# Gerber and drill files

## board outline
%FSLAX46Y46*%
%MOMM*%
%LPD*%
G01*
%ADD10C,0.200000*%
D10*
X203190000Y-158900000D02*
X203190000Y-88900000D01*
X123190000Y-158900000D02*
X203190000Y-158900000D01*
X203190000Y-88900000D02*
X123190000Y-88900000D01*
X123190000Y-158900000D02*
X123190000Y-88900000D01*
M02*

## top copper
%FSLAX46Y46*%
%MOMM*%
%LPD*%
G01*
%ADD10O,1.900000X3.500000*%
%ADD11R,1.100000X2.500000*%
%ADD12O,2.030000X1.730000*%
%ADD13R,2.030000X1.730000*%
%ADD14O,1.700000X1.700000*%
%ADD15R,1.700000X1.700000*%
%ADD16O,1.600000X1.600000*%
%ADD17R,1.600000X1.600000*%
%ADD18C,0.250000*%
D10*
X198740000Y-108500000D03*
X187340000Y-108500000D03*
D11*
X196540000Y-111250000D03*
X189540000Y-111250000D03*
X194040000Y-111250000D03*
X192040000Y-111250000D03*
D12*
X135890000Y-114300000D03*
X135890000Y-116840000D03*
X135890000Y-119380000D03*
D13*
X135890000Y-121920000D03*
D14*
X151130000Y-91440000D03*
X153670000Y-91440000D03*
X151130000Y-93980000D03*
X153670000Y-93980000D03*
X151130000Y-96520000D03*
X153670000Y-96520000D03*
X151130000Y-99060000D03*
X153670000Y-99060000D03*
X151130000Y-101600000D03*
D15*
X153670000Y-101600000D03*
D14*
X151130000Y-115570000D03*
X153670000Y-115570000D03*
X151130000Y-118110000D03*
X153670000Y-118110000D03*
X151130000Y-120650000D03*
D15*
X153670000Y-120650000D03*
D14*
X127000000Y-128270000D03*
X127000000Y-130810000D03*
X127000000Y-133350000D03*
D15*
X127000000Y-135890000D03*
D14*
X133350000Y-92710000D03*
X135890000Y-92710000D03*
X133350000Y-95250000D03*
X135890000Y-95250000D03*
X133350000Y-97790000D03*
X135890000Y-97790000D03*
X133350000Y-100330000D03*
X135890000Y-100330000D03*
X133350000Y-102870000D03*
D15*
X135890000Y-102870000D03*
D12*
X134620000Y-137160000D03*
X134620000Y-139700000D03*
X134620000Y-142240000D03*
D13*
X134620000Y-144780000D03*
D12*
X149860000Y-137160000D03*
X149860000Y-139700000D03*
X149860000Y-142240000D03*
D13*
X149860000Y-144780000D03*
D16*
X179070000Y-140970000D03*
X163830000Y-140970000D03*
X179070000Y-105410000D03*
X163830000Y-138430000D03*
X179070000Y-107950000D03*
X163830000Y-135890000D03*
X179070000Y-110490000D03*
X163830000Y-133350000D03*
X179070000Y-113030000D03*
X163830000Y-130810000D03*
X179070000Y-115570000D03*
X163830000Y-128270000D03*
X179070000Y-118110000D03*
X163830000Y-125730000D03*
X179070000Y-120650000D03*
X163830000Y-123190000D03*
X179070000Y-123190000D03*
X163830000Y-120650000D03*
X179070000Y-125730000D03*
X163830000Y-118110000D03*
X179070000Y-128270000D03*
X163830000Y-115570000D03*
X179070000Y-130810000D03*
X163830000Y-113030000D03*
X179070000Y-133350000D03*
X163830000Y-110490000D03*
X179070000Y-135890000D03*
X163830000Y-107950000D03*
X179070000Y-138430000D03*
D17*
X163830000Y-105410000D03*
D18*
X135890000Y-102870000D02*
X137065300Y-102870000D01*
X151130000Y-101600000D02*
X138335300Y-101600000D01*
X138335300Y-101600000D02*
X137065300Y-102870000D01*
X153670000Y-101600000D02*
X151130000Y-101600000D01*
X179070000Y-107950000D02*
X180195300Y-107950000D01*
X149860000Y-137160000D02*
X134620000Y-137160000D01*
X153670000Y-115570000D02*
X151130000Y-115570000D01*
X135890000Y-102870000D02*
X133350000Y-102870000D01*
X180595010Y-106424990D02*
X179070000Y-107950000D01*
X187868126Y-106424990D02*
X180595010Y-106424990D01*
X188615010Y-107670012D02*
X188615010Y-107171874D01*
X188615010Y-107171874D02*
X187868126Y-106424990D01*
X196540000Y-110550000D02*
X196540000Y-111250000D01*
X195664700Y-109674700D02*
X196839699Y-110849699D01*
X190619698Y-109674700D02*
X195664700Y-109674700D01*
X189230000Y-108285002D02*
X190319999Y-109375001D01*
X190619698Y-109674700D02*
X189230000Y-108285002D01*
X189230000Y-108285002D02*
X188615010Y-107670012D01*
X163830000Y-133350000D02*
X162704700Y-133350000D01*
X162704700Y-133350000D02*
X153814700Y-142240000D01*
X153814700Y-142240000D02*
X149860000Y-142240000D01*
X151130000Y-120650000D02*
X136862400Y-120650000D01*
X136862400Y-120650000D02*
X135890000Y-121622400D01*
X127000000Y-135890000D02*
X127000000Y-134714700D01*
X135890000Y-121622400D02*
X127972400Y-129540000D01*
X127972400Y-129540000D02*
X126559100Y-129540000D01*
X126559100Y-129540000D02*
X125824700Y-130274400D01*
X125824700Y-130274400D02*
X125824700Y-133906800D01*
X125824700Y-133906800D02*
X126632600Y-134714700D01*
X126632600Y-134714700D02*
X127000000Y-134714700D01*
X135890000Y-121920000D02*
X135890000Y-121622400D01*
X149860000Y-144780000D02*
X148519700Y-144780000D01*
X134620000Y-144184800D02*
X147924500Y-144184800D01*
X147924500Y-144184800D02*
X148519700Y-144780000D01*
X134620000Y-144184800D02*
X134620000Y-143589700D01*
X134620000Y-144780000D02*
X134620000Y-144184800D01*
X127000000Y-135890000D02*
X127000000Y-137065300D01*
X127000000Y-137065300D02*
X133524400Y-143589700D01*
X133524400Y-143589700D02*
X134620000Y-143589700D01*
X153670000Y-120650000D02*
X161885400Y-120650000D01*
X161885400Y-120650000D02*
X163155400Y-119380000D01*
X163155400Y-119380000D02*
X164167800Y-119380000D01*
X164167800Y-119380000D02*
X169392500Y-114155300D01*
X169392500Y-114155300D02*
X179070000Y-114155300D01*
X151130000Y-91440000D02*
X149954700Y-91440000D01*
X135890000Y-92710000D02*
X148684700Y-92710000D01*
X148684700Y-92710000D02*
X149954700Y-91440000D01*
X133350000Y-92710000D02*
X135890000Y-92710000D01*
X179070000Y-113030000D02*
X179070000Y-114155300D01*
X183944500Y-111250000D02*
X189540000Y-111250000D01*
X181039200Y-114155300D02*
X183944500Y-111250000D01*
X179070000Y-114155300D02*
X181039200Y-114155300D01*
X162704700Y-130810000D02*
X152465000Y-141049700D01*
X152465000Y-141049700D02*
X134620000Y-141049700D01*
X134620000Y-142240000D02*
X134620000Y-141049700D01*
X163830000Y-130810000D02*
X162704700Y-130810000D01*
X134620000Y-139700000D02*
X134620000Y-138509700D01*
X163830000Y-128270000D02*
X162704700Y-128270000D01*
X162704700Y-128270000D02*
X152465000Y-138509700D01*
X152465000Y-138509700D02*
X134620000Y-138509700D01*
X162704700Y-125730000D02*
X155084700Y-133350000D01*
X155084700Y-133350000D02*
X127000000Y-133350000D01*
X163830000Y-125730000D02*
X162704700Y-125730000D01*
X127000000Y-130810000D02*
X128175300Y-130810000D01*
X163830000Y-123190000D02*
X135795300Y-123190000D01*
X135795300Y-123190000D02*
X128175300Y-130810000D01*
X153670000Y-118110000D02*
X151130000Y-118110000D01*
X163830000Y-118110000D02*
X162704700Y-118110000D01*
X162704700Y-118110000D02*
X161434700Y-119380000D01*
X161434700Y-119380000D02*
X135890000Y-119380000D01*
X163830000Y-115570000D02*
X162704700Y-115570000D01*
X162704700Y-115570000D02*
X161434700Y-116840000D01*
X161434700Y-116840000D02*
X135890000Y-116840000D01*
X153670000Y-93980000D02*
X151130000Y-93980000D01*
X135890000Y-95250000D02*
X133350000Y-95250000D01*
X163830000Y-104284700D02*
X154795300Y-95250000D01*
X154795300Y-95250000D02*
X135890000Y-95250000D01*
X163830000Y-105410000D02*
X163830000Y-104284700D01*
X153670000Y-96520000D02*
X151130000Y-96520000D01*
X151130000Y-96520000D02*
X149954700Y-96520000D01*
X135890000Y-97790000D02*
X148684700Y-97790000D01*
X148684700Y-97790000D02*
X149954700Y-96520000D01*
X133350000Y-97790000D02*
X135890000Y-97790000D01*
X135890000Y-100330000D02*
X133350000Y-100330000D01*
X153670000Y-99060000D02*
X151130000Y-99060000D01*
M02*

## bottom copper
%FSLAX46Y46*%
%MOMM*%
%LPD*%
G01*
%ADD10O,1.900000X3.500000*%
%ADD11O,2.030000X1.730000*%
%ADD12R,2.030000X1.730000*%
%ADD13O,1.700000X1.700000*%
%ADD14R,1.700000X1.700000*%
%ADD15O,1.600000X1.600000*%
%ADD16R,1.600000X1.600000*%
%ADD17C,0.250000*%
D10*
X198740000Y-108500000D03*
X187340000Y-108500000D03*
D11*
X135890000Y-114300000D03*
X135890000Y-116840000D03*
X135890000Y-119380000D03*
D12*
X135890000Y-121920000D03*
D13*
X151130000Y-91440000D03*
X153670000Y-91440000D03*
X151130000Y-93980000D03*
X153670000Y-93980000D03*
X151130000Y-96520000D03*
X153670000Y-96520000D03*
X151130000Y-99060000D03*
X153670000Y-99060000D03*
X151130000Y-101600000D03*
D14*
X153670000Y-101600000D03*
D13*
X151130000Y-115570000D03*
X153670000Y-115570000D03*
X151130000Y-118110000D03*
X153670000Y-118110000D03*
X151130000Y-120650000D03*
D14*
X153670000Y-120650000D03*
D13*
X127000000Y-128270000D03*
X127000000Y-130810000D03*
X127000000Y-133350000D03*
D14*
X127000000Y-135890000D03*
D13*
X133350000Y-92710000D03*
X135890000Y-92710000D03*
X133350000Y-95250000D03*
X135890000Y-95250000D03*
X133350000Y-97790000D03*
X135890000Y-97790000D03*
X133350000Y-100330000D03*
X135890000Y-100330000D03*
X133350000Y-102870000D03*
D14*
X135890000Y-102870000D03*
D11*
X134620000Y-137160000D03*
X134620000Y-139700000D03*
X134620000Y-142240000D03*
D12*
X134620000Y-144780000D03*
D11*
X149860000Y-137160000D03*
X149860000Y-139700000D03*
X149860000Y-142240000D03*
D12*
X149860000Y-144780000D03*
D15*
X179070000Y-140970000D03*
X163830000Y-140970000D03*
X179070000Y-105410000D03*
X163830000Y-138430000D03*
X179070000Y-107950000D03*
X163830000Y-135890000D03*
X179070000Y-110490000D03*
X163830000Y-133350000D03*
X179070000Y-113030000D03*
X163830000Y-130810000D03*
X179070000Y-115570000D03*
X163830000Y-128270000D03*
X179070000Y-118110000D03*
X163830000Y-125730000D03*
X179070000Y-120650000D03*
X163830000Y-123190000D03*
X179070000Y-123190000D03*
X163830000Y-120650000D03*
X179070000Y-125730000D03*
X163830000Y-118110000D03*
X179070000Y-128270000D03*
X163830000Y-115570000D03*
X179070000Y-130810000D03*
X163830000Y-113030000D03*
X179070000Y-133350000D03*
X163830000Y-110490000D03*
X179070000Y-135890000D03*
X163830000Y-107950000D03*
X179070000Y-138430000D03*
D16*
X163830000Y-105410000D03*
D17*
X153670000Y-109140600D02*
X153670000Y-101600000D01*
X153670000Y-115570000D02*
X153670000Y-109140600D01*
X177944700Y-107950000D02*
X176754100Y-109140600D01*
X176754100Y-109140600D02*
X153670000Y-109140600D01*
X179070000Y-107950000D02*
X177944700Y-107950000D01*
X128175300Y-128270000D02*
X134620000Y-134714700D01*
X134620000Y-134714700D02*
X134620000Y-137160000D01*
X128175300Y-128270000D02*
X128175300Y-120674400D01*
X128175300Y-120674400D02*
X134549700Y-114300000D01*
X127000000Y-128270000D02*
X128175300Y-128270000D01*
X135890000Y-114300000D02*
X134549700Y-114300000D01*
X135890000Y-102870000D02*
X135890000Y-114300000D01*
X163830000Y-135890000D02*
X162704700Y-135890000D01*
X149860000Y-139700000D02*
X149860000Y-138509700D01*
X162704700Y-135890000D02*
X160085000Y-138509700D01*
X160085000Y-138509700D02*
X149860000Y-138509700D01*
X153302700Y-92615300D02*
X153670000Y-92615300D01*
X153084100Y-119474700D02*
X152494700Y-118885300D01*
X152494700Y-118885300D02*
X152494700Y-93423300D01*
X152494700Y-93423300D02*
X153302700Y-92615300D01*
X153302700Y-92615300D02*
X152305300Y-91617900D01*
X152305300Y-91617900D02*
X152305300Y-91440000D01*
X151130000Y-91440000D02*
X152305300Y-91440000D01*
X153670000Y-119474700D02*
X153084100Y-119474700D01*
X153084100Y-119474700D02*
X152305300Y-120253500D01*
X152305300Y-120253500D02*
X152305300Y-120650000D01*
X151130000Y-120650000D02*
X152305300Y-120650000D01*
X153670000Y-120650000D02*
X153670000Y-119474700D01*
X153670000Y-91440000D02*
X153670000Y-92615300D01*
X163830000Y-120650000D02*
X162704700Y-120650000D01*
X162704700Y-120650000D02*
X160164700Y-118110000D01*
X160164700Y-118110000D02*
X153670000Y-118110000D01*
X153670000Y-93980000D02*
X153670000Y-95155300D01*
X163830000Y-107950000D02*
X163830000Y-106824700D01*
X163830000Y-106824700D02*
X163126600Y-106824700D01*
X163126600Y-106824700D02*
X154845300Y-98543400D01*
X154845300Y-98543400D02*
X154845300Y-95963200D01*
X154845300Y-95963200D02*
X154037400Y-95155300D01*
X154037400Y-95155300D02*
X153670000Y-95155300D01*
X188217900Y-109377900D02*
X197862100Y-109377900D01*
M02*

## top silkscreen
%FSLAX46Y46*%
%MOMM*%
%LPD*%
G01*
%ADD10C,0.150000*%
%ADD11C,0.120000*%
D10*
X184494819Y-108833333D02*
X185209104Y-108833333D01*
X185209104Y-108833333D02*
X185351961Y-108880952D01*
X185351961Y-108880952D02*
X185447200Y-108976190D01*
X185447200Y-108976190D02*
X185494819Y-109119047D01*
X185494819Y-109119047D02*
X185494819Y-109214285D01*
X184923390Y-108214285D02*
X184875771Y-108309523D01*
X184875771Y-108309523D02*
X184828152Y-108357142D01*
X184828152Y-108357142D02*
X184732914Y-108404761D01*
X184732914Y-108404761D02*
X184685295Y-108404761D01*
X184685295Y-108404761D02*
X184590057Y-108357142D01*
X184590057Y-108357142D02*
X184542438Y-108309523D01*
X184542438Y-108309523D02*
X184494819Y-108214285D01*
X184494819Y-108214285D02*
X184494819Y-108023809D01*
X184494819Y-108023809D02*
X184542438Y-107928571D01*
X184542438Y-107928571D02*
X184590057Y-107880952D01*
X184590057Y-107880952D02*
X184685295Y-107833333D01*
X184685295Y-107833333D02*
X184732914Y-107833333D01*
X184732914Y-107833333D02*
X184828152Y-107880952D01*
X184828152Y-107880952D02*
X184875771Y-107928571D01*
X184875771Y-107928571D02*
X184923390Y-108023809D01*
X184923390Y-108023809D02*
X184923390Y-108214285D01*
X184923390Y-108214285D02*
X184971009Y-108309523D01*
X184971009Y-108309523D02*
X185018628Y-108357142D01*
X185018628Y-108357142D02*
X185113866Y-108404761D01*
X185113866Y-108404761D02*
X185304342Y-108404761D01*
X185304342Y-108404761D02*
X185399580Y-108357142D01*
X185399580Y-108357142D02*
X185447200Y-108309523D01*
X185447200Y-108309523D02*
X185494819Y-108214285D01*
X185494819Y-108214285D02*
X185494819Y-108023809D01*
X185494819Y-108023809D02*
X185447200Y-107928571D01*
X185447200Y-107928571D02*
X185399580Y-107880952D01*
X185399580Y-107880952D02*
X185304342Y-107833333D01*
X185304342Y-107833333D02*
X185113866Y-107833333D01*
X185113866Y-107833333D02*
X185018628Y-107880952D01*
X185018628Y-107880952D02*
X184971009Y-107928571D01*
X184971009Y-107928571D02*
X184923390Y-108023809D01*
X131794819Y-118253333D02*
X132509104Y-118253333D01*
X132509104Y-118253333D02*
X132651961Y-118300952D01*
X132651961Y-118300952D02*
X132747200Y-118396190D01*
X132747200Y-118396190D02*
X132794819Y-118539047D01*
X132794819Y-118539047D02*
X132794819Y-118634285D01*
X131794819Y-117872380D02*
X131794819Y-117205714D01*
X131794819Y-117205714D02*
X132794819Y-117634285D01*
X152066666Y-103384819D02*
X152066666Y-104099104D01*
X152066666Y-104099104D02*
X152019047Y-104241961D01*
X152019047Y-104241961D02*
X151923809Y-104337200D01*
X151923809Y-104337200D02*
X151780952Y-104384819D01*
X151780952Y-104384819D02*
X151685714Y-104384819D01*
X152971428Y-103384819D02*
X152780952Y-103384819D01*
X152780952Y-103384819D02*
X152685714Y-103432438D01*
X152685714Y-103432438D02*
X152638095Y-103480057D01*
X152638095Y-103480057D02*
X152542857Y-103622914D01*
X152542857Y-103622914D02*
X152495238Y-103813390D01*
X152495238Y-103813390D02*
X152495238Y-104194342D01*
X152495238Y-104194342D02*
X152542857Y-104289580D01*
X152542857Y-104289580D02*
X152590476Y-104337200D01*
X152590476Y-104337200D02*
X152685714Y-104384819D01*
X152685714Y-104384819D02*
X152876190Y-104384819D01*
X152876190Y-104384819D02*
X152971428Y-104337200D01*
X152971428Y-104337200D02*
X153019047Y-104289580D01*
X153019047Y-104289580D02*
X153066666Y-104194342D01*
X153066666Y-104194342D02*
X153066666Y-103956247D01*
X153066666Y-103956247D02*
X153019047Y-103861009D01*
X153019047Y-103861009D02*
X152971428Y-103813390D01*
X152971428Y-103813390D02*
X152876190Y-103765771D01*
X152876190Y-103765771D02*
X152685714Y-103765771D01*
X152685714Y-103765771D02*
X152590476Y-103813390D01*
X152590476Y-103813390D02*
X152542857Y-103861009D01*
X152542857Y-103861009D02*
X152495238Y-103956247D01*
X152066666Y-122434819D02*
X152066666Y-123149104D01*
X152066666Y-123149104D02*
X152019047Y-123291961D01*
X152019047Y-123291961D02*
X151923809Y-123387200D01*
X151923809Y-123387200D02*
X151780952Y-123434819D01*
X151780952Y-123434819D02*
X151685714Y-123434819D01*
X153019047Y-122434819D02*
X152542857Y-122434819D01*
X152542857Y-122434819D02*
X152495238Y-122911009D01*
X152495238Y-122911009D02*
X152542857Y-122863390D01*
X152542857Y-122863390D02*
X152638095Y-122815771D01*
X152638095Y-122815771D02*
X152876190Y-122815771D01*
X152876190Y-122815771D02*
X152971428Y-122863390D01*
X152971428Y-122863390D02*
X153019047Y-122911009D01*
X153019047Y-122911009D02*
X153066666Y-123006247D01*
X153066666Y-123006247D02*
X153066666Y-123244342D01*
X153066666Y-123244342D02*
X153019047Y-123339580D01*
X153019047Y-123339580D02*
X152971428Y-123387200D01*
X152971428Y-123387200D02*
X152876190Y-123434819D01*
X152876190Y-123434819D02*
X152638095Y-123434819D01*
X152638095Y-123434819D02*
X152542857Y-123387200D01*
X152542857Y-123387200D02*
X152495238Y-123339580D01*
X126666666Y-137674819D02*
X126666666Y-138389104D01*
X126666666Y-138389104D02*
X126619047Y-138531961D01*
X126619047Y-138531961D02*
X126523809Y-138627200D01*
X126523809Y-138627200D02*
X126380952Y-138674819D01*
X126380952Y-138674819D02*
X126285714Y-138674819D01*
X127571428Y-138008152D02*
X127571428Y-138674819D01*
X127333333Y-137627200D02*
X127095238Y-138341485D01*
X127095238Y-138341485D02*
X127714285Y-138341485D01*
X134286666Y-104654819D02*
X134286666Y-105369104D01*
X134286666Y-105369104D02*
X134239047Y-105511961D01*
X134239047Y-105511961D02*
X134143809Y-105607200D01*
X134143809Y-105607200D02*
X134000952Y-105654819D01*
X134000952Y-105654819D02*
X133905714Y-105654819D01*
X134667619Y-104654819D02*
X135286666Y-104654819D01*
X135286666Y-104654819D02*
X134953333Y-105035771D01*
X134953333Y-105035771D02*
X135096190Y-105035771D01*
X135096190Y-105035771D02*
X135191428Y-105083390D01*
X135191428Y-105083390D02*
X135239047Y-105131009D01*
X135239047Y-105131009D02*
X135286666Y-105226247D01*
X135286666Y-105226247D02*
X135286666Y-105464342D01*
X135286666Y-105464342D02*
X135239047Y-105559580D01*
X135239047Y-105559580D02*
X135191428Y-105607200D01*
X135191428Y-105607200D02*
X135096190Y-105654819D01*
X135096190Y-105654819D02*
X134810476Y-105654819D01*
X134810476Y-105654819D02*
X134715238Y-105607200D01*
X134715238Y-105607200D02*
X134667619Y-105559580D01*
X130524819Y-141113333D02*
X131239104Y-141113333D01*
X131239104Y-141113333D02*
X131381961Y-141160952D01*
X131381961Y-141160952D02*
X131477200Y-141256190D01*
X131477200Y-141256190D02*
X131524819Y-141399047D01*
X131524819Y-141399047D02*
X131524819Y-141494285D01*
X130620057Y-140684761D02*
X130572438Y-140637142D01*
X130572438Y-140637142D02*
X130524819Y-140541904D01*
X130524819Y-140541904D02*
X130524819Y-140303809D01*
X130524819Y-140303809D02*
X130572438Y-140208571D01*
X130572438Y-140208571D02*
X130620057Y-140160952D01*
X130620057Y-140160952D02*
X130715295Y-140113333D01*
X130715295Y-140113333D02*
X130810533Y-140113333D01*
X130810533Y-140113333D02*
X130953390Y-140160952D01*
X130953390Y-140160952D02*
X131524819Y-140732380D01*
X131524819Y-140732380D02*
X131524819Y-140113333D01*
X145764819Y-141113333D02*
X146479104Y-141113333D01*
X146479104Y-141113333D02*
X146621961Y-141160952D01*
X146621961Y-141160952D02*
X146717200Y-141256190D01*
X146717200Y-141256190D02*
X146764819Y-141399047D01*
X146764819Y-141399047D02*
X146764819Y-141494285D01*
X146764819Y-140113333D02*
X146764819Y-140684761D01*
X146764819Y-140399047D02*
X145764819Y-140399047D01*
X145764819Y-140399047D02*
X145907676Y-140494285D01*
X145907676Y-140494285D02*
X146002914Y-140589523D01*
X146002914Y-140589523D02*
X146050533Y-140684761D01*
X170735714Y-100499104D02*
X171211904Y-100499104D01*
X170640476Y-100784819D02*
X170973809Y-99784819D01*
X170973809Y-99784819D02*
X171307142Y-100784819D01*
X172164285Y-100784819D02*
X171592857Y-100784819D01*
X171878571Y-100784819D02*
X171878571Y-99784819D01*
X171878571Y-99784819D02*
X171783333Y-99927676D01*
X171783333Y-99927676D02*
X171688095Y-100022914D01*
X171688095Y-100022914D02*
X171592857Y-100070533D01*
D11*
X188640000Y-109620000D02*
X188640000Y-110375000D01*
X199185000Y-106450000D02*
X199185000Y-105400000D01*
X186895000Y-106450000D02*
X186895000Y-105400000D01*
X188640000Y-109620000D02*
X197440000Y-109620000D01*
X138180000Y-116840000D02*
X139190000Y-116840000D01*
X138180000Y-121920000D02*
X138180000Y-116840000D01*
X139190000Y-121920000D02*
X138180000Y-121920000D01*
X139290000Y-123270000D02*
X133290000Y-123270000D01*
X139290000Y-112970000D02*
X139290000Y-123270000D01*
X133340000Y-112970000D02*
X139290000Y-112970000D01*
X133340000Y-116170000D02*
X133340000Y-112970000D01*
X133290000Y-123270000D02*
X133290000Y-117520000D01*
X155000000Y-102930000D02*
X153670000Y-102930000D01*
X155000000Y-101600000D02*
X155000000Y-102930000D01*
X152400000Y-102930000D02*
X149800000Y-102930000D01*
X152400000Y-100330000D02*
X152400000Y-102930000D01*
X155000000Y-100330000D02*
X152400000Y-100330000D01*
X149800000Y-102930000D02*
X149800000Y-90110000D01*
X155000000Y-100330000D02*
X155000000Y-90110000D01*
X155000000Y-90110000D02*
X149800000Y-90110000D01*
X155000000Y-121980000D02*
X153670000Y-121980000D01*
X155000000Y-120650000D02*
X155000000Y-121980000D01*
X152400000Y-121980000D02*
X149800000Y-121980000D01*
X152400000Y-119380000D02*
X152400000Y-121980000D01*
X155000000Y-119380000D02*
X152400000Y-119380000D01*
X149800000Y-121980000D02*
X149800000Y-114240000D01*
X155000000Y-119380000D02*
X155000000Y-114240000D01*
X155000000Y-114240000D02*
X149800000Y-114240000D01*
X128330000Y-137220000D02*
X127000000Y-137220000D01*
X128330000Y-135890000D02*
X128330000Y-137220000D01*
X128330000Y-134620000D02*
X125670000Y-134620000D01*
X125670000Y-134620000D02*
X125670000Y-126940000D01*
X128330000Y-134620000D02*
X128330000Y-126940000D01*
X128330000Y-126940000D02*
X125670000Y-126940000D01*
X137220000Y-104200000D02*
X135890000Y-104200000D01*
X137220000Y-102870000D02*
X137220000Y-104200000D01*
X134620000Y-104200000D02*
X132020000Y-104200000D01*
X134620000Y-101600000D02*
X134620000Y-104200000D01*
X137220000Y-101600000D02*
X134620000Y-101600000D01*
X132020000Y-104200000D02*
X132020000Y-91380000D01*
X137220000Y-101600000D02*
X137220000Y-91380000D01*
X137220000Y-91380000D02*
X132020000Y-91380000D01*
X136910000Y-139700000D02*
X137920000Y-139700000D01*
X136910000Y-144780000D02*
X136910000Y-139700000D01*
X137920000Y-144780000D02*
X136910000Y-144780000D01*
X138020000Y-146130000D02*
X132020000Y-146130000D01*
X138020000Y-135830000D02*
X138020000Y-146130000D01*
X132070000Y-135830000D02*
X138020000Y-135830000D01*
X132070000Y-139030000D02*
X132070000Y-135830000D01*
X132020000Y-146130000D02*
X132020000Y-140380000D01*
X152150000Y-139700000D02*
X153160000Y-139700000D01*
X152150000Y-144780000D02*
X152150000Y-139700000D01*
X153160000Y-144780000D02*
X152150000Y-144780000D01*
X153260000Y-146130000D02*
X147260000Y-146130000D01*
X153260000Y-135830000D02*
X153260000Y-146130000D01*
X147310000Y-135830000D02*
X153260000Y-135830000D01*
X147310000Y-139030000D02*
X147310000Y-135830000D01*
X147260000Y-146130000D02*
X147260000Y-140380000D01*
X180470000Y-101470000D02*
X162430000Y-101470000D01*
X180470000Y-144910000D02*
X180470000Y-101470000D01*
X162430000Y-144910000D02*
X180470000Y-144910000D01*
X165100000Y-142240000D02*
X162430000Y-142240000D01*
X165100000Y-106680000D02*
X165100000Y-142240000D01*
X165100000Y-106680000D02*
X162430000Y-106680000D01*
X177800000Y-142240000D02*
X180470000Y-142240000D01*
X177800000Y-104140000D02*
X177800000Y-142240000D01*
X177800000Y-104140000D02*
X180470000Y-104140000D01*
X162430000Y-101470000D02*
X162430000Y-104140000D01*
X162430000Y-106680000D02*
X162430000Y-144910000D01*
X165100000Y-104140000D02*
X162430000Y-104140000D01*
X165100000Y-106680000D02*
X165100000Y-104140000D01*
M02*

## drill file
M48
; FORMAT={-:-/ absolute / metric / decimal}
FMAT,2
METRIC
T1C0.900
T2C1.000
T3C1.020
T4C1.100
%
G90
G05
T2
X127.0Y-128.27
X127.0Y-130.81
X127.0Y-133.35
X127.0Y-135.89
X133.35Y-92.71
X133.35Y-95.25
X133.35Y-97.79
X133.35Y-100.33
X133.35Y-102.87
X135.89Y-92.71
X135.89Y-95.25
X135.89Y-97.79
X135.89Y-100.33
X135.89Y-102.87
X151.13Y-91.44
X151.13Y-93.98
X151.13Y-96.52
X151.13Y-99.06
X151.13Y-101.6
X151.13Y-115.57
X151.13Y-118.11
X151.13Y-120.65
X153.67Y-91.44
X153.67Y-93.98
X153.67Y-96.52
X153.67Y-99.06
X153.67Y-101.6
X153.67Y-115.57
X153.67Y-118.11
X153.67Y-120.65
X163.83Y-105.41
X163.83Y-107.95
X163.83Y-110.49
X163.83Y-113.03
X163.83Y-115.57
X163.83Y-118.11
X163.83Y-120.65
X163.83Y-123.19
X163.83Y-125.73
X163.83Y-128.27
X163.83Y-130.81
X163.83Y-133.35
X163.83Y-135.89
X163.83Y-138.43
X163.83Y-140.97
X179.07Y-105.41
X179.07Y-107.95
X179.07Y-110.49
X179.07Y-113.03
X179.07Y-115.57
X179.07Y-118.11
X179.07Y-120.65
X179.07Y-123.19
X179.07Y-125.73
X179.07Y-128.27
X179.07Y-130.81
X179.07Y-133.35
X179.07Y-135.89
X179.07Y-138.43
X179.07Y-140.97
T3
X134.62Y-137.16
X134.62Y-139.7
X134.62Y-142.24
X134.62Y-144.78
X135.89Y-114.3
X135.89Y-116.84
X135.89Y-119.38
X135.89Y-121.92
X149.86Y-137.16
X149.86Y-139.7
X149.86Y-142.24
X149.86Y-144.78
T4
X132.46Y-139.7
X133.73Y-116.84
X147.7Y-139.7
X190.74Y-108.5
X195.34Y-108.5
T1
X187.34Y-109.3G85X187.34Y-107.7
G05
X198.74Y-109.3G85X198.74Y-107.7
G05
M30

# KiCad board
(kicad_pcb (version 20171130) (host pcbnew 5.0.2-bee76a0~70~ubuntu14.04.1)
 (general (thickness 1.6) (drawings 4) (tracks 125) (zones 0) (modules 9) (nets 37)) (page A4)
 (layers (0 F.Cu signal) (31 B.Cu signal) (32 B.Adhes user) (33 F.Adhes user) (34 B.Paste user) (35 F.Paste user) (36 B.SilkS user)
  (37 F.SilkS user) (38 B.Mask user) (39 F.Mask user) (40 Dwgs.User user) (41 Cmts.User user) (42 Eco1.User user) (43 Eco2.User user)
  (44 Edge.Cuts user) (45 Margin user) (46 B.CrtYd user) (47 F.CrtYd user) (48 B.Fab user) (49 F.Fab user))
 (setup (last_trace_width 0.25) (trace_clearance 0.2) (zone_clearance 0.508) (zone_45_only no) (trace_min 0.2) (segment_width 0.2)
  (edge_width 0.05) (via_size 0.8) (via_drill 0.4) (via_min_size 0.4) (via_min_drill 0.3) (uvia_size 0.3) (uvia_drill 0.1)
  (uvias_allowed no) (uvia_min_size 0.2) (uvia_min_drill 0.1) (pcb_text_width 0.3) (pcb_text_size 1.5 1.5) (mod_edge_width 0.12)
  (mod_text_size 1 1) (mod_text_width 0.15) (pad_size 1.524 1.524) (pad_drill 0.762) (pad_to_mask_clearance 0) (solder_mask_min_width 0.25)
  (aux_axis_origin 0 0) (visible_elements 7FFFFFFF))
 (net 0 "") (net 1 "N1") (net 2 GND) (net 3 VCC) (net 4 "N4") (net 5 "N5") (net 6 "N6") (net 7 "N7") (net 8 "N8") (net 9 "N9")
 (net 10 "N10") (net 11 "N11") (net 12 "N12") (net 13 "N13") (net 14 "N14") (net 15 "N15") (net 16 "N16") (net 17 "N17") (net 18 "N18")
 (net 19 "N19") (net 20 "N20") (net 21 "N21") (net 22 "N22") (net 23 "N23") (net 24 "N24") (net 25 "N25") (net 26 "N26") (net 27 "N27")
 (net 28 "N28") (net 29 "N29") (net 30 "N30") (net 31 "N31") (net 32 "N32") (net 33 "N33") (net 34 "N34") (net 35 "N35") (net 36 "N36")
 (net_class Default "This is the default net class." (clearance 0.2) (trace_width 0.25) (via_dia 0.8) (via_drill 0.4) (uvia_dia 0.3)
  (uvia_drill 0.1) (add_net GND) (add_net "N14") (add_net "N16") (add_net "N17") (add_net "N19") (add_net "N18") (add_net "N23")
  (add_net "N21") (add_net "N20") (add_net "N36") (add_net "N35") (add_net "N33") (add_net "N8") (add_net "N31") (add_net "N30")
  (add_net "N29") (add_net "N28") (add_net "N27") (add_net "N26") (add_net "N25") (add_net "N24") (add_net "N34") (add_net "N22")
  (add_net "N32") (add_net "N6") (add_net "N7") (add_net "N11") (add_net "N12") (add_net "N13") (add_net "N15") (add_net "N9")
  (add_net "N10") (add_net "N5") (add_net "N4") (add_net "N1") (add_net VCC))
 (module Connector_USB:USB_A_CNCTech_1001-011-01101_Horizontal (layer F.Cu) (at 193.04 101.6 90)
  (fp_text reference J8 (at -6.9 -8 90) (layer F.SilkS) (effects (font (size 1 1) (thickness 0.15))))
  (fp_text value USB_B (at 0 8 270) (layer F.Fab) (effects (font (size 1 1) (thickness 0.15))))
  (fp_line (start -8.02 -4.4) (end -8.775 -4.4) (layer F.SilkS) (width 0.12))
  (fp_line (start -4.85 6.145) (end -3.8 6.145) (layer F.SilkS) (width 0.12))
  (fp_line (start -4.85 -6.145) (end -3.8 -6.145) (layer F.SilkS) (width 0.12))
  (fp_line (start -8.02 -4.4) (end -8.02 4.4) (layer F.SilkS) (width 0.12))
  (pad "" np_thru_hole circle (at -6.9 2.3 90) (size 1.1 1.1) (drill 1.1) (layers *.Cu *.Mask))
  (pad "" np_thru_hole circle (at -6.9 -2.3 90) (size 1.1 1.1) (drill 1.1) (layers *.Cu *.Mask))
  (pad 5 thru_hole oval (at -6.9 5.7 90) (size 3.5 1.9) (drill oval 2.5 0.9) (layers *.Cu *.Mask) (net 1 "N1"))
  (pad 5 thru_hole oval (at -6.9 -5.7 90) (size 3.5 1.9) (drill oval 2.5 0.9) (layers *.Cu *.Mask) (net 1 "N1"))
  (pad 4 smd rect (at -9.65 3.5 90) (size 2.5 1.1) (layers F.Cu F.Paste F.Mask) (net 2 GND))
  (pad 1 smd rect (at -9.65 -3.5 90) (size 2.5 1.1) (layers F.Cu F.Paste F.Mask) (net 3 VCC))
  (pad 3 smd rect (at -9.65 1 90) (size 2.5 1.1) (layers F.Cu F.Paste F.Mask) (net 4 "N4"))
  (pad 2 smd rect (at -9.65 -1 90) (size 2.5 1.1) (layers F.Cu F.Paste F.Mask) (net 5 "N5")))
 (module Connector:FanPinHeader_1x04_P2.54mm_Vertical (layer F.Cu) (at 135.89 121.92 90)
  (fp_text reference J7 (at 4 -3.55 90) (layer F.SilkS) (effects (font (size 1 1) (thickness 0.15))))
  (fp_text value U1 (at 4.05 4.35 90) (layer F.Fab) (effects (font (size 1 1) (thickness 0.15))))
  (fp_line (start 5.08 2.29) (end 5.08 3.3) (layer F.SilkS) (width 0.12))
  (fp_line (start 0 2.29) (end 5.08 2.29) (layer F.SilkS) (width 0.12))
  (fp_line (start 0 3.3) (end 0 2.29) (layer F.SilkS) (width 0.12))
  (fp_line (start -1.35 3.4) (end -1.35 -2.6) (layer F.SilkS) (width 0.12))
  (fp_line (start 8.95 3.4) (end -1.35 3.4) (layer F.SilkS) (width 0.12))
  (fp_line (start 8.95 -2.55) (end 8.95 3.4) (layer F.SilkS) (width 0.12))
  (fp_line (start 5.75 -2.55) (end 8.95 -2.55) (layer F.SilkS) (width 0.12))
  (fp_line (start -1.35 -2.6) (end 4.4 -2.6) (layer F.SilkS) (width 0.12))
  (pad "" np_thru_hole circle (at 5.08 -2.16 180) (size 1.1 1.1) (drill 1.1) (layers *.Cu *.Mask))
  (pad 4 thru_hole oval (at 7.62 0 180) (size 2.03 1.73) (drill 1.02) (layers *.Cu *.Mask) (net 2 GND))
  (pad 3 thru_hole oval (at 5.08 0 180) (size 2.03 1.73) (drill 1.02) (layers *.Cu *.Mask) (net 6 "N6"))
  (pad 2 thru_hole oval (at 2.54 0 180) (size 2.03 1.73) (drill 1.02) (layers *.Cu *.Mask) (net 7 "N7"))
  (pad 1 thru_hole rect (at 0 0 180) (size 2.03 1.73) (drill 1.02) (layers *.Cu *.Mask) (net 3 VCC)))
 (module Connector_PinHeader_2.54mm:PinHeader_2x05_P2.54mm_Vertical (layer F.Cu) (at 153.67 101.6 180)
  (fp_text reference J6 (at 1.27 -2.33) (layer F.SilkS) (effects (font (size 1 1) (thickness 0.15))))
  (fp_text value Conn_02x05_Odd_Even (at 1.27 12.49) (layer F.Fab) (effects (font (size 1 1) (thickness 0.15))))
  (fp_line (start -1.33 -1.33) (end 0 -1.33) (layer F.SilkS) (width 0.12))
  (fp_line (start -1.33 0) (end -1.33 -1.33) (layer F.SilkS) (width 0.12))
  (fp_line (start 1.27 -1.33) (end 3.87 -1.33) (layer F.SilkS) (width 0.12))
  (fp_line (start 1.27 1.27) (end 1.27 -1.33) (layer F.SilkS) (width 0.12))
  (fp_line (start -1.33 1.27) (end 1.27 1.27) (layer F.SilkS) (width 0.12))
  (fp_line (start 3.87 -1.33) (end 3.87 11.49) (layer F.SilkS) (width 0.12))
  (fp_line (start -1.33 1.27) (end -1.33 11.49) (layer F.SilkS) (width 0.12))
  (fp_line (start -1.33 11.49) (end 3.87 11.49) (layer F.SilkS) (width 0.12))
  (pad 10 thru_hole oval (at 2.54 10.16 180) (size 1.7 1.7) (drill 1) (layers *.Cu *.Mask) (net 3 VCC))
  (pad 9 thru_hole oval (at 0 10.16 180) (size 1.7 1.7) (drill 1) (layers *.Cu *.Mask) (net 3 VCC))
  (pad 8 thru_hole oval (at 2.54 7.62 180) (size 1.7 1.7) (drill 1) (layers *.Cu *.Mask) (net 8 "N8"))
  (pad 7 thru_hole oval (at 0 7.62 180) (size 1.7 1.7) (drill 1) (layers *.Cu *.Mask) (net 8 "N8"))
  (pad 6 thru_hole oval (at 2.54 5.08 180) (size 1.7 1.7) (drill 1) (layers *.Cu *.Mask) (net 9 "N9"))
  (pad 5 thru_hole oval (at 0 5.08 180) (size 1.7 1.7) (drill 1) (layers *.Cu *.Mask) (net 9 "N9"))
  (pad 4 thru_hole oval (at 2.54 2.54 180) (size 1.7 1.7) (drill 1) (layers *.Cu *.Mask) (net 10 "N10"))
  (pad 3 thru_hole oval (at 0 2.54 180) (size 1.7 1.7) (drill 1) (layers *.Cu *.Mask) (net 10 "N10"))
  (pad 2 thru_hole oval (at 2.54 0 180) (size 1.7 1.7) (drill 1) (layers *.Cu *.Mask) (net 2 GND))
  (pad 1 thru_hole rect (at 0 0 180) (size 1.7 1.7) (drill 1) (layers *.Cu *.Mask) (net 2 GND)))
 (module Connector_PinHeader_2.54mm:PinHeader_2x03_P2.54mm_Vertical (layer F.Cu) (at 153.67 120.65 180)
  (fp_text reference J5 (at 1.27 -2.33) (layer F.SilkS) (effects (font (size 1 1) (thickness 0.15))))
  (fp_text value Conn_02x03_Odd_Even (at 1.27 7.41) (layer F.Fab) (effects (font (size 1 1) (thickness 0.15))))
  (fp_line (start -1.33 -1.33) (end 0 -1.33) (layer F.SilkS) (width 0.12))
  (fp_line (start -1.33 0) (end -1.33 -1.33) (layer F.SilkS) (width 0.12))
  (fp_line (start 1.27 -1.33) (end 3.87 -1.33) (layer F.SilkS) (width 0.12))
  (fp_line (start 1.27 1.27) (end 1.27 -1.33) (layer F.SilkS) (width 0.12))
  (fp_line (start -1.33 1.27) (end 1.27 1.27) (layer F.SilkS) (width 0.12))
  (fp_line (start 3.87 -1.33) (end 3.87 6.41) (layer F.SilkS) (width 0.12))
  (fp_line (start -1.33 1.27) (end -1.33 6.41) (layer F.SilkS) (width 0.12))
  (fp_line (start -1.33 6.41) (end 3.87 6.41) (layer F.SilkS) (width 0.12))
  (pad 6 thru_hole oval (at 2.54 5.08 180) (size 1.7 1.7) (drill 1) (layers *.Cu *.Mask) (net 2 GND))
  (pad 5 thru_hole oval (at 0 5.08 180) (size 1.7 1.7) (drill 1) (layers *.Cu *.Mask) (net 2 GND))
  (pad 4 thru_hole oval (at 2.54 2.54 180) (size 1.7 1.7) (drill 1) (layers *.Cu *.Mask) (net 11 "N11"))
  (pad 3 thru_hole oval (at 0 2.54 180) (size 1.7 1.7) (drill 1) (layers *.Cu *.Mask) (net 11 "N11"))
  (pad 2 thru_hole oval (at 2.54 0 180) (size 1.7 1.7) (drill 1) (layers *.Cu *.Mask) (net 3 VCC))
  (pad 1 thru_hole rect (at 0 0 180) (size 1.7 1.7) (drill 1) (layers *.Cu *.Mask) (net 3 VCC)))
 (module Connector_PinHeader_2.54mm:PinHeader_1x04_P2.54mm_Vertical (layer F.Cu) (at 127 135.89 180)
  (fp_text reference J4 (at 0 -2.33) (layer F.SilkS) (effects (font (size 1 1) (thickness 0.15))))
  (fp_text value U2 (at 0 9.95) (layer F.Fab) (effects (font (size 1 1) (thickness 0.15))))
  (fp_line (start -1.33 -1.33) (end 0 -1.33) (layer F.SilkS) (width 0.12))
  (fp_line (start -1.33 0) (end -1.33 -1.33) (layer F.SilkS) (width 0.12))
  (fp_line (start -1.33 1.27) (end 1.33 1.27) (layer F.SilkS) (width 0.12))
  (fp_line (start 1.33 1.27) (end 1.33 8.95) (layer F.SilkS) (width 0.12))
  (fp_line (start -1.33 1.27) (end -1.33 8.95) (layer F.SilkS) (width 0.12))
  (fp_line (start -1.33 8.95) (end 1.33 8.95) (layer F.SilkS) (width 0.12))
  (pad 4 thru_hole oval (at 0 7.62 180) (size 1.7 1.7) (drill 1) (layers *.Cu *.Mask) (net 2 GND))
  (pad 3 thru_hole oval (at 0 5.08 180) (size 1.7 1.7) (drill 1) (layers *.Cu *.Mask) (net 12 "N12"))
  (pad 2 thru_hole oval (at 0 2.54 180) (size 1.7 1.7) (drill 1) (layers *.Cu *.Mask) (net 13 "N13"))
  (pad 1 thru_hole rect (at 0 0 180) (size 1.7 1.7) (drill 1) (layers *.Cu *.Mask) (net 3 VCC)))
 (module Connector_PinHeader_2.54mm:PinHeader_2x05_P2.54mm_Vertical (layer F.Cu) (at 135.89 102.87 180)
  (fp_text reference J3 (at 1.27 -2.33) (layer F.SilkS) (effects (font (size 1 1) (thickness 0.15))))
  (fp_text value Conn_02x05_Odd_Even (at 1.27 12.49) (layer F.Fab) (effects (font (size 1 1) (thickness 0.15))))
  (fp_line (start -1.33 -1.33) (end 0 -1.33) (layer F.SilkS) (width 0.12))
  (fp_line (start -1.33 0) (end -1.33 -1.33) (layer F.SilkS) (width 0.12))
  (fp_line (start 1.27 -1.33) (end 3.87 -1.33) (layer F.SilkS) (width 0.12))
  (fp_line (start 1.27 1.27) (end 1.27 -1.33) (layer F.SilkS) (width 0.12))
  (fp_line (start -1.33 1.27) (end 1.27 1.27) (layer F.SilkS) (width 0.12))
  (fp_line (start 3.87 -1.33) (end 3.87 11.49) (layer F.SilkS) (width 0.12))
  (fp_line (start -1.33 1.27) (end -1.33 11.49) (layer F.SilkS) (width 0.12))
  (fp_line (start -1.33 11.49) (end 3.87 11.49) (layer F.SilkS) (width 0.12))
  (pad 10 thru_hole oval (at 2.54 10.16 180) (size 1.7 1.7) (drill 1) (layers *.Cu *.Mask) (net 3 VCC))
  (pad 9 thru_hole oval (at 0 10.16 180) (size 1.7 1.7) (drill 1) (layers *.Cu *.Mask) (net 3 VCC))
  (pad 8 thru_hole oval (at 2.54 7.62 180) (size 1.7 1.7) (drill 1) (layers *.Cu *.Mask) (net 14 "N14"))
  (pad 7 thru_hole oval (at 0 7.62 180) (size 1.7 1.7) (drill 1) (layers *.Cu *.Mask) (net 14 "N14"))
  (pad 6 thru_hole oval (at 2.54 5.08 180) (size 1.7 1.7) (drill 1) (layers *.Cu *.Mask) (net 9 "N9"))
  (pad 5 thru_hole oval (at 0 5.08 180) (size 1.7 1.7) (drill 1) (layers *.Cu *.Mask) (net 9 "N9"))
  (pad 4 thru_hole oval (at 2.54 2.54 180) (size 1.7 1.7) (drill 1) (layers *.Cu *.Mask) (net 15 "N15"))
  (pad 3 thru_hole oval (at 0 2.54 180) (size 1.7 1.7) (drill 1) (layers *.Cu *.Mask) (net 15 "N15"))
  (pad 2 thru_hole oval (at 2.54 0 180) (size 1.7 1.7) (drill 1) (layers *.Cu *.Mask) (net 2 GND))
  (pad 1 thru_hole rect (at 0 0 180) (size 1.7 1.7) (drill 1) (layers *.Cu *.Mask) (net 2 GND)))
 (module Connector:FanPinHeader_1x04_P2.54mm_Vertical (layer F.Cu) (at 134.62 144.78 90)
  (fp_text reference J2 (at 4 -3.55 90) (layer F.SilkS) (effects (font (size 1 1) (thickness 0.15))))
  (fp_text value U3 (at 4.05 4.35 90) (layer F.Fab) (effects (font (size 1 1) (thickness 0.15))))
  (fp_line (start 5.08 2.29) (end 5.08 3.3) (layer F.SilkS) (width 0.12))
  (fp_line (start 0 2.29) (end 5.08 2.29) (layer F.SilkS) (width 0.12))
  (fp_line (start 0 3.3) (end 0 2.29) (layer F.SilkS) (width 0.12))
  (fp_line (start -1.35 3.4) (end -1.35 -2.6) (layer F.SilkS) (width 0.12))
  (fp_line (start 8.95 3.4) (end -1.35 3.4) (layer F.SilkS) (width 0.12))
  (fp_line (start 8.95 -2.55) (end 8.95 3.4) (layer F.SilkS) (width 0.12))
  (fp_line (start 5.75 -2.55) (end 8.95 -2.55) (layer F.SilkS) (width 0.12))
  (fp_line (start -1.35 -2.6) (end 4.4 -2.6) (layer F.SilkS) (width 0.12))
  (pad "" np_thru_hole circle (at 5.08 -2.16 180) (size 1.1 1.1) (drill 1.1) (layers *.Cu *.Mask))
  (pad 4 thru_hole oval (at 7.62 0 180) (size 2.03 1.73) (drill 1.02) (layers *.Cu *.Mask) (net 2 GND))
  (pad 3 thru_hole oval (at 5.08 0 180) (size 2.03 1.73) (drill 1.02) (layers *.Cu *.Mask) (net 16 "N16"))
  (pad 2 thru_hole oval (at 2.54 0 180) (size 2.03 1.73) (drill 1.02) (layers *.Cu *.Mask) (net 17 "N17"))
  (pad 1 thru_hole rect (at 0 0 180) (size 2.03 1.73) (drill 1.02) (layers *.Cu *.Mask) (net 3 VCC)))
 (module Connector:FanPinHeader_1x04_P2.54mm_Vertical (layer F.Cu) (at 149.86 144.78 90)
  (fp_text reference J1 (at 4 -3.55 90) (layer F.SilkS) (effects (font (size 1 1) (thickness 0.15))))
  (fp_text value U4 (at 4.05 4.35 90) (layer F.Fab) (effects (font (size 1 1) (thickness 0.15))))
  (fp_line (start 5.08 2.29) (end 5.08 3.3) (layer F.SilkS) (width 0.12))
  (fp_line (start 0 2.29) (end 5.08 2.29) (layer F.SilkS) (width 0.12))
  (fp_line (start 0 3.3) (end 0 2.29) (layer F.SilkS) (width 0.12))
  (fp_line (start -1.35 3.4) (end -1.35 -2.6) (layer F.SilkS) (width 0.12))
  (fp_line (start 8.95 3.4) (end -1.35 3.4) (layer F.SilkS) (width 0.12))
  (fp_line (start 8.95 -2.55) (end 8.95 3.4) (layer F.SilkS) (width 0.12))
  (fp_line (start 5.75 -2.55) (end 8.95 -2.55) (layer F.SilkS) (width 0.12))
  (fp_line (start -1.35 -2.6) (end 4.4 -2.6) (layer F.SilkS) (width 0.12))
  (pad "" np_thru_hole circle (at 5.08 -2.16 180) (size 1.1 1.1) (drill 1.1) (layers *.Cu *.Mask))
  (pad 4 thru_hole oval (at 7.62 0 180) (size 2.03 1.73) (drill 1.02) (layers *.Cu *.Mask) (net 2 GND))
  (pad 3 thru_hole oval (at 5.08 0 180) (size 2.03 1.73) (drill 1.02) (layers *.Cu *.Mask) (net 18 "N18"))
  (pad 2 thru_hole oval (at 2.54 0 180) (size 2.03 1.73) (drill 1.02) (layers *.Cu *.Mask) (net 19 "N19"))
  (pad 1 thru_hole rect (at 0 0 180) (size 2.03 1.73) (drill 1.02) (layers *.Cu *.Mask) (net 3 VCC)))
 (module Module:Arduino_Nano (layer F.Cu) (at 163.83 105.41)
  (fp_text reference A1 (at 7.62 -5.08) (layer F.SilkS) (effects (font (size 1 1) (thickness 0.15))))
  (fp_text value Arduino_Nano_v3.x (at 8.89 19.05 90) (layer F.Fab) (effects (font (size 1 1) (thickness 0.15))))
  (fp_line (start 16.64 -3.94) (end -1.4 -3.94) (layer F.SilkS) (width 0.12))
  (fp_line (start 16.64 39.5) (end 16.64 -3.94) (layer F.SilkS) (width 0.12))
  (fp_line (start -1.4 39.5) (end 16.64 39.5) (layer F.SilkS) (width 0.12))
  (fp_line (start 1.27 36.83) (end -1.4 36.83) (layer F.SilkS) (width 0.12))
  (fp_line (start 1.27 1.27) (end 1.27 36.83) (layer F.SilkS) (width 0.12))
  (fp_line (start 1.27 1.27) (end -1.4 1.27) (layer F.SilkS) (width 0.12))
  (fp_line (start 13.97 36.83) (end 16.64 36.83) (layer F.SilkS) (width 0.12))
  (fp_line (start 13.97 -1.27) (end 13.97 36.83) (layer F.SilkS) (width 0.12))
  (fp_line (start 13.97 -1.27) (end 16.64 -1.27) (layer F.SilkS) (width 0.12))
  (fp_line (start -1.4 -3.94) (end -1.4 -1.27) (layer F.SilkS) (width 0.12))
  (fp_line (start -1.4 1.27) (end -1.4 39.5) (layer F.SilkS) (width 0.12))
  (fp_line (start 1.27 -1.27) (end -1.4 -1.27) (layer F.SilkS) (width 0.12))
  (fp_line (start 1.27 1.27) (end 1.27 -1.27) (layer F.SilkS) (width 0.12))
  (pad 16 thru_hole oval (at 15.24 35.56) (size 1.6 1.6) (drill 1) (layers *.Cu *.Mask) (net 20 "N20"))
  (pad 15 thru_hole oval (at 0 35.56) (size 1.6 1.6) (drill 1) (layers *.Cu *.Mask) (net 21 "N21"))
  (pad 30 thru_hole oval (at 15.24 0) (size 1.6 1.6) (drill 1) (layers *.Cu *.Mask) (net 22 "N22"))
  (pad 14 thru_hole oval (at 0 33.02) (size 1.6 1.6) (drill 1) (layers *.Cu *.Mask) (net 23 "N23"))
  (pad 29 thru_hole oval (at 15.24 2.54) (size 1.6 1.6) (drill 1) (layers *.Cu *.Mask) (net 2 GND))
  (pad 13 thru_hole oval (at 0 30.48) (size 1.6 1.6) (drill 1) (layers *.Cu *.Mask) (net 18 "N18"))
  (pad 28 thru_hole oval (at 15.24 5.08) (size 1.6 1.6) (drill 1) (layers *.Cu *.Mask) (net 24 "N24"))
  (pad 12 thru_hole oval (at 0 27.94) (size 1.6 1.6) (drill 1) (layers *.Cu *.Mask) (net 19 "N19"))
  (pad 27 thru_hole oval (at 15.24 7.62) (size 1.6 1.6) (drill 1) (layers *.Cu *.Mask) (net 3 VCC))
  (pad 11 thru_hole oval (at 0 25.4) (size 1.6 1.6) (drill 1) (layers *.Cu *.Mask) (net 17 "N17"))
  (pad 26 thru_hole oval (at 15.24 10.16) (size 1.6 1.6) (drill 1) (layers *.Cu *.Mask) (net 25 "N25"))
  (pad 10 thru_hole oval (at 0 22.86) (size 1.6 1.6) (drill 1) (layers *.Cu *.Mask) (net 16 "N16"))
  (pad 25 thru_hole oval (at 15.24 12.7) (size 1.6 1.6) (drill 1) (layers *.Cu *.Mask) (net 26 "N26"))
  (pad 9 thru_hole oval (at 0 20.32) (size 1.6 1.6) (drill 1) (layers *.Cu *.Mask) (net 13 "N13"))
  (pad 24 thru_hole oval (at 15.24 15.24) (size 1.6 1.6) (drill 1) (layers *.Cu *.Mask) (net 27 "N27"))
  (pad 8 thru_hole oval (at 0 17.78) (size 1.6 1.6) (drill 1) (layers *.Cu *.Mask) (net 12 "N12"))
  (pad 23 thru_hole oval (at 15.24 17.78) (size 1.6 1.6) (drill 1) (layers *.Cu *.Mask) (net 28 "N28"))
  (pad 7 thru_hole oval (at 0 15.24) (size 1.6 1.6) (drill 1) (layers *.Cu *.Mask) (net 11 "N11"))
  (pad 22 thru_hole oval (at 15.24 20.32) (size 1.6 1.6) (drill 1) (layers *.Cu *.Mask) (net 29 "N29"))
  (pad 6 thru_hole oval (at 0 12.7) (size 1.6 1.6) (drill 1) (layers *.Cu *.Mask) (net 7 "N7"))
  (pad 21 thru_hole oval (at 15.24 22.86) (size 1.6 1.6) (drill 1) (layers *.Cu *.Mask) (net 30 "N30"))
  (pad 5 thru_hole oval (at 0 10.16) (size 1.6 1.6) (drill 1) (layers *.Cu *.Mask) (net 6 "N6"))
  (pad 20 thru_hole oval (at 15.24 25.4) (size 1.6 1.6) (drill 1) (layers *.Cu *.Mask) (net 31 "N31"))
  (pad 4 thru_hole oval (at 0 7.62) (size 1.6 1.6) (drill 1) (layers *.Cu *.Mask) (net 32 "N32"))
  (pad 19 thru_hole oval (at 15.24 27.94) (size 1.6 1.6) (drill 1) (layers *.Cu *.Mask) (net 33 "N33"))
  (pad 3 thru_hole oval (at 0 5.08) (size 1.6 1.6) (drill 1) (layers *.Cu *.Mask) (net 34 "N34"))
  (pad 18 thru_hole oval (at 15.24 30.48) (size 1.6 1.6) (drill 1) (layers *.Cu *.Mask) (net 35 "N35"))
  (pad 2 thru_hole oval (at 0 2.54) (size 1.6 1.6) (drill 1) (layers *.Cu *.Mask) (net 8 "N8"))
  (pad 17 thru_hole oval (at 15.24 33.02) (size 1.6 1.6) (drill 1) (layers *.Cu *.Mask) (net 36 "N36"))
  (pad 1 thru_hole rect (at 0 0) (size 1.6 1.6) (drill 1) (layers *.Cu *.Mask) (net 14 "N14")))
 (gr_line (start 203.19 158.9) (end 203.19 88.9) (layer Edge.Cuts) (width 0.2))
 (gr_line (start 123.19 158.9) (end 203.19 158.9) (layer Edge.Cuts) (width 0.2))
 (gr_line (start 203.19 88.9) (end 123.19 88.9) (layer Edge.Cuts) (width 0.2))
 (gr_line (start 123.19 158.9) (end 123.19 88.9) (layer Edge.Cuts) (width 0.2))
 (segment (start 135.89 102.87) (end 137.0653 102.87) (width 0.25) (layer F.Cu) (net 2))
 (segment (start 151.13 101.6) (end 138.3353 101.6) (width 0.25) (layer F.Cu) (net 2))
 (segment (start 138.3353 101.6) (end 137.0653 102.87) (width 0.25) (layer F.Cu) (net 2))
 (segment (start 153.67 101.6) (end 151.13 101.6) (width 0.25) (layer F.Cu) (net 2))
 (segment (start 153.67 109.1406) (end 153.67 101.6) (width 0.25) (layer B.Cu) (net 2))
 (segment (start 153.67 115.57) (end 153.67 109.1406) (width 0.25) (layer B.Cu) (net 2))
 (segment (start 177.9447 107.95) (end 176.7541 109.1406) (width 0.25) (layer B.Cu) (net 2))
 (segment (start 176.7541 109.1406) (end 153.67 109.1406) (width 0.25) (layer B.Cu) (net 2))
 (segment (start 179.07 107.95) (end 177.9447 107.95) (width 0.25) (layer B.Cu) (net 2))
 (segment (start 128.1753 128.27) (end 134.62 134.7147) (width 0.25) (layer B.Cu) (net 2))
 (segment (start 134.62 134.7147) (end 134.62 137.16) (width 0.25) (layer B.Cu) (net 2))
 (segment (start 128.1753 128.27) (end 128.1753 120.6744) (width 0.25) (layer B.Cu) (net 2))
 (segment (start 128.1753 120.6744) (end 134.5497 114.3) (width 0.25) (layer B.Cu) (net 2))
 (segment (start 127 128.27) (end 128.1753 128.27) (width 0.25) (layer B.Cu) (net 2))
 (segment (start 135.89 114.3) (end 134.5497 114.3) (width 0.25) (layer B.Cu) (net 2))
 (segment (start 135.89 102.87) (end 135.89 114.3) (width 0.25) (layer B.Cu) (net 2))
 (segment (start 179.07 107.95) (end 180.1953 107.95) (width 0.25) (layer F.Cu) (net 2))
 (segment (start 149.86 137.16) (end 134.62 137.16) (width 0.25) (layer F.Cu) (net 2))
 (segment (start 153.67 115.57) (end 151.13 115.57) (width 0.25) (layer F.Cu) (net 2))
 (segment (start 135.89 102.87) (end 133.35 102.87) (width 0.25) (layer F.Cu) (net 2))
 (segment (start 180.59501 106.42499) (end 179.07 107.95) (width 0.25) (layer F.Cu) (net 2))
 (segment (start 187.868126 106.42499) (end 180.59501 106.42499) (width 0.25) (layer F.Cu) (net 2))
 (segment (start 188.61501 107.670012) (end 188.61501 107.171874) (width 0.25) (layer F.Cu) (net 2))
 (segment (start 188.61501 107.171874) (end 187.868126 106.42499) (width 0.25) (layer F.Cu) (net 2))
 (segment (start 196.54 110.55) (end 196.54 111.25) (width 0.25) (layer F.Cu) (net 2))
 (segment (start 195.6647 109.6747) (end 196.839699 110.849699) (width 0.25) (layer F.Cu) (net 2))
 (segment (start 190.619698 109.6747) (end 195.6647 109.6747) (width 0.25) (layer F.Cu) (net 2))
 (segment (start 189.23 108.285002) (end 190.319999 109.375001) (width 0.25) (layer F.Cu) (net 2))
 (segment (start 190.619698 109.6747) (end 189.23 108.285002) (width 0.25) (layer F.Cu) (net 2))
 (segment (start 189.23 108.285002) (end 188.61501 107.670012) (width 0.25) (layer F.Cu) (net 2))
 (segment (start 163.83 135.89) (end 162.7047 135.89) (width 0.25) (layer B.Cu) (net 18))
 (segment (start 149.86 139.7) (end 149.86 138.5097) (width 0.25) (layer B.Cu) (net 18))
 (segment (start 162.7047 135.89) (end 160.085 138.5097) (width 0.25) (layer B.Cu) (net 18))
 (segment (start 160.085 138.5097) (end 149.86 138.5097) (width 0.25) (layer B.Cu) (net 18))
 (segment (start 163.83 133.35) (end 162.7047 133.35) (width 0.25) (layer F.Cu) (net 19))
 (segment (start 162.7047 133.35) (end 153.8147 142.24) (width 0.25) (layer F.Cu) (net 19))
 (segment (start 153.8147 142.24) (end 149.86 142.24) (width 0.25) (layer F.Cu) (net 19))
 (segment (start 151.13 120.65) (end 136.8624 120.65) (width 0.25) (layer F.Cu) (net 3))
 (segment (start 136.8624 120.65) (end 135.89 121.6224) (width 0.25) (layer F.Cu) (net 3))
 (segment (start 127 135.89) (end 127 134.7147) (width 0.25) (layer F.Cu) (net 3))
 (segment (start 135.89 121.6224) (end 127.9724 129.54) (width 0.25) (layer F.Cu) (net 3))
 (segment (start 127.9724 129.54) (end 126.5591 129.54) (width 0.25) (layer F.Cu) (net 3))
 (segment (start 126.5591 129.54) (end 125.8247 130.2744) (width 0.25) (layer F.Cu) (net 3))
 (segment (start 125.8247 130.2744) (end 125.8247 133.9068) (width 0.25) (layer F.Cu) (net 3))
 (segment (start 125.8247 133.9068) (end 126.6326 134.7147) (width 0.25) (layer F.Cu) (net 3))
 (segment (start 126.6326 134.7147) (end 127 134.7147) (width 0.25) (layer F.Cu) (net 3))
 (segment (start 135.89 121.92) (end 135.89 121.6224) (width 0.25) (layer F.Cu) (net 3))
 (segment (start 153.3027 92.6153) (end 153.67 92.6153) (width 0.25) (layer B.Cu) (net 3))
 (segment (start 153.0841 119.4747) (end 152.4947 118.8853) (width 0.25) (layer B.Cu) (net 3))
 (segment (start 152.4947 118.8853) (end 152.4947 93.4233) (width 0.25) (layer B.Cu) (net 3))
 (segment (start 152.4947 93.4233) (end 153.3027 92.6153) (width 0.25) (layer B.Cu) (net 3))
 (segment (start 153.3027 92.6153) (end 152.3053 91.6179) (width 0.25) (layer B.Cu) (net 3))
 (segment (start 152.3053 91.6179) (end 152.3053 91.44) (width 0.25) (layer B.Cu) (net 3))
 (segment (start 151.13 91.44) (end 152.3053 91.44) (width 0.25) (layer B.Cu) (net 3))
 (segment (start 153.67 119.4747) (end 153.0841 119.4747) (width 0.25) (layer B.Cu) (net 3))
 (segment (start 153.0841 119.4747) (end 152.3053 120.2535) (width 0.25) (layer B.Cu) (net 3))
 (segment (start 152.3053 120.2535) (end 152.3053 120.65) (width 0.25) (layer B.Cu) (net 3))
 (segment (start 151.13 120.65) (end 152.3053 120.65) (width 0.25) (layer B.Cu) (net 3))
 (segment (start 149.86 144.78) (end 148.5197 144.78) (width 0.25) (layer F.Cu) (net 3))
 (segment (start 134.62 144.1848) (end 147.9245 144.1848) (width 0.25) (layer F.Cu) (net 3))
 (segment (start 147.9245 144.1848) (end 148.5197 144.78) (width 0.25) (layer F.Cu) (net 3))
 (segment (start 134.62 144.1848) (end 134.62 143.5897) (width 0.25) (layer F.Cu) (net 3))
 (segment (start 134.62 144.78) (end 134.62 144.1848) (width 0.25) (layer F.Cu) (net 3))
 (segment (start 127 135.89) (end 127 137.0653) (width 0.25) (layer F.Cu) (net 3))
 (segment (start 127 137.0653) (end 133.5244 143.5897) (width 0.25) (layer F.Cu) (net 3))
 (segment (start 133.5244 143.5897) (end 134.62 143.5897) (width 0.25) (layer F.Cu) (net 3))
 (segment (start 153.67 120.65) (end 161.8854 120.65) (width 0.25) (layer F.Cu) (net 3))
 (segment (start 161.8854 120.65) (end 163.1554 119.38) (width 0.25) (layer F.Cu) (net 3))
 (segment (start 163.1554 119.38) (end 164.1678 119.38) (width 0.25) (layer F.Cu) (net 3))
 (segment (start 164.1678 119.38) (end 169.3925 114.1553) (width 0.25) (layer F.Cu) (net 3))
 (segment (start 169.3925 114.1553) (end 179.07 114.1553) (width 0.25) (layer F.Cu) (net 3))
 (segment (start 153.67 120.65) (end 153.67 119.4747) (width 0.25) (layer B.Cu) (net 3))
 (segment (start 153.67 91.44) (end 153.67 92.6153) (width 0.25) (layer B.Cu) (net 3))
 (segment (start 151.13 91.44) (end 149.9547 91.44) (width 0.25) (layer F.Cu) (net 3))
 (segment (start 135.89 92.71) (end 148.6847 92.71) (width 0.25) (layer F.Cu) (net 3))
 (segment (start 148.6847 92.71) (end 149.9547 91.44) (width 0.25) (layer F.Cu) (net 3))
 (segment (start 133.35 92.71) (end 135.89 92.71) (width 0.25) (layer F.Cu) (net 3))
 (segment (start 179.07 113.03) (end 179.07 114.1553) (width 0.25) (layer F.Cu) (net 3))
 (segment (start 183.9445 111.25) (end 189.54 111.25) (width 0.25) (layer F.Cu) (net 3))
 (segment (start 181.0392 114.1553) (end 183.9445 111.25) (width 0.25) (layer F.Cu) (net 3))
 (segment (start 179.07 114.1553) (end 181.0392 114.1553) (width 0.25) (layer F.Cu) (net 3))
 (segment (start 162.7047 130.81) (end 152.465 141.0497) (width 0.25) (layer F.Cu) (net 17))
 (segment (start 152.465 141.0497) (end 134.62 141.0497) (width 0.25) (layer F.Cu) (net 17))
 (segment (start 134.62 142.24) (end 134.62 141.0497) (width 0.25) (layer F.Cu) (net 17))
 (segment (start 163.83 130.81) (end 162.7047 130.81) (width 0.25) (layer F.Cu) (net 17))
 (segment (start 134.62 139.7) (end 134.62 138.5097) (width 0.25) (layer F.Cu) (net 16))
 (segment (start 163.83 128.27) (end 162.7047 128.27) (width 0.25) (layer F.Cu) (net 16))
 (segment (start 162.7047 128.27) (end 152.465 138.5097) (width 0.25) (layer F.Cu) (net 16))
 (segment (start 152.465 138.5097) (end 134.62 138.5097) (width 0.25) (layer F.Cu) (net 16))
 (segment (start 162.7047 125.73) (end 155.0847 133.35) (width 0.25) (layer F.Cu) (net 13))
 (segment (start 155.0847 133.35) (end 127 133.35) (width 0.25) (layer F.Cu) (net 13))
 (segment (start 163.83 125.73) (end 162.7047 125.73) (width 0.25) (layer F.Cu) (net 13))
 (segment (start 127 130.81) (end 128.1753 130.81) (width 0.25) (layer F.Cu) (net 12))
 (segment (start 163.83 123.19) (end 135.7953 123.19) (width 0.25) (layer F.Cu) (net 12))
 (segment (start 135.7953 123.19) (end 128.1753 130.81) (width 0.25) (layer F.Cu) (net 12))
 (segment (start 153.67 118.11) (end 151.13 118.11) (width 0.25) (layer F.Cu) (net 11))
 (segment (start 163.83 120.65) (end 162.7047 120.65) (width 0.25) (layer B.Cu) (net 11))
 (segment (start 162.7047 120.65) (end 160.1647 118.11) (width 0.25) (layer B.Cu) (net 11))
 (segment (start 160.1647 118.11) (end 153.67 118.11) (width 0.25) (layer B.Cu) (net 11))
 (segment (start 163.83 118.11) (end 162.7047 118.11) (width 0.25) (layer F.Cu) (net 7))
 (segment (start 162.7047 118.11) (end 161.4347 119.38) (width 0.25) (layer F.Cu) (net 7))
 (segment (start 161.4347 119.38) (end 135.89 119.38) (width 0.25) (layer F.Cu) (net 7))
 (segment (start 163.83 115.57) (end 162.7047 115.57) (width 0.25) (layer F.Cu) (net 6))
 (segment (start 162.7047 115.57) (end 161.4347 116.84) (width 0.25) (layer F.Cu) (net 6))
 (segment (start 161.4347 116.84) (end 135.89 116.84) (width 0.25) (layer F.Cu) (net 6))
 (segment (start 153.67 93.98) (end 153.67 95.1553) (width 0.25) (layer B.Cu) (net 8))
 (segment (start 163.83 107.95) (end 163.83 106.8247) (width 0.25) (layer B.Cu) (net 8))
 (segment (start 163.83 106.8247) (end 163.1266 106.8247) (width 0.25) (layer B.Cu) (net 8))
 (segment (start 163.1266 106.8247) (end 154.8453 98.5434) (width 0.25) (layer B.Cu) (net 8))
 (segment (start 154.8453 98.5434) (end 154.8453 95.9632) (width 0.25) (layer B.Cu) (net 8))
 (segment (start 154.8453 95.9632) (end 154.0374 95.1553) (width 0.25) (layer B.Cu) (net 8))
 (segment (start 154.0374 95.1553) (end 153.67 95.1553) (width 0.25) (layer B.Cu) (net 8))
 (segment (start 153.67 93.98) (end 151.13 93.98) (width 0.25) (layer F.Cu) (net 8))
 (segment (start 135.89 95.25) (end 133.35 95.25) (width 0.25) (layer F.Cu) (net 14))
 (segment (start 163.83 104.2847) (end 154.7953 95.25) (width 0.25) (layer F.Cu) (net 14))
 (segment (start 154.7953 95.25) (end 135.89 95.25) (width 0.25) (layer F.Cu) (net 14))
 (segment (start 163.83 105.41) (end 163.83 104.2847) (width 0.25) (layer F.Cu) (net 14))
 (segment (start 153.67 96.52) (end 151.13 96.52) (width 0.25) (layer F.Cu) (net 9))
 (segment (start 151.13 96.52) (end 149.9547 96.52) (width 0.25) (layer F.Cu) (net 9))
 (segment (start 135.89 97.79) (end 148.6847 97.79) (width 0.25) (layer F.Cu) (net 9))
 (segment (start 148.6847 97.79) (end 149.9547 96.52) (width 0.25) (layer F.Cu) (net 9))
 (segment (start 133.35 97.79) (end 135.89 97.79) (width 0.25) (layer F.Cu) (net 9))
 (segment (start 135.89 100.33) (end 133.35 100.33) (width 0.25) (layer F.Cu) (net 15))
 (segment (start 153.67 99.06) (end 151.13 99.06) (width 0.25) (layer F.Cu) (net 10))
 (segment (start 188.2179 109.3779) (end 197.8621 109.3779) (width 0.25) (layer B.Cu) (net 1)))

